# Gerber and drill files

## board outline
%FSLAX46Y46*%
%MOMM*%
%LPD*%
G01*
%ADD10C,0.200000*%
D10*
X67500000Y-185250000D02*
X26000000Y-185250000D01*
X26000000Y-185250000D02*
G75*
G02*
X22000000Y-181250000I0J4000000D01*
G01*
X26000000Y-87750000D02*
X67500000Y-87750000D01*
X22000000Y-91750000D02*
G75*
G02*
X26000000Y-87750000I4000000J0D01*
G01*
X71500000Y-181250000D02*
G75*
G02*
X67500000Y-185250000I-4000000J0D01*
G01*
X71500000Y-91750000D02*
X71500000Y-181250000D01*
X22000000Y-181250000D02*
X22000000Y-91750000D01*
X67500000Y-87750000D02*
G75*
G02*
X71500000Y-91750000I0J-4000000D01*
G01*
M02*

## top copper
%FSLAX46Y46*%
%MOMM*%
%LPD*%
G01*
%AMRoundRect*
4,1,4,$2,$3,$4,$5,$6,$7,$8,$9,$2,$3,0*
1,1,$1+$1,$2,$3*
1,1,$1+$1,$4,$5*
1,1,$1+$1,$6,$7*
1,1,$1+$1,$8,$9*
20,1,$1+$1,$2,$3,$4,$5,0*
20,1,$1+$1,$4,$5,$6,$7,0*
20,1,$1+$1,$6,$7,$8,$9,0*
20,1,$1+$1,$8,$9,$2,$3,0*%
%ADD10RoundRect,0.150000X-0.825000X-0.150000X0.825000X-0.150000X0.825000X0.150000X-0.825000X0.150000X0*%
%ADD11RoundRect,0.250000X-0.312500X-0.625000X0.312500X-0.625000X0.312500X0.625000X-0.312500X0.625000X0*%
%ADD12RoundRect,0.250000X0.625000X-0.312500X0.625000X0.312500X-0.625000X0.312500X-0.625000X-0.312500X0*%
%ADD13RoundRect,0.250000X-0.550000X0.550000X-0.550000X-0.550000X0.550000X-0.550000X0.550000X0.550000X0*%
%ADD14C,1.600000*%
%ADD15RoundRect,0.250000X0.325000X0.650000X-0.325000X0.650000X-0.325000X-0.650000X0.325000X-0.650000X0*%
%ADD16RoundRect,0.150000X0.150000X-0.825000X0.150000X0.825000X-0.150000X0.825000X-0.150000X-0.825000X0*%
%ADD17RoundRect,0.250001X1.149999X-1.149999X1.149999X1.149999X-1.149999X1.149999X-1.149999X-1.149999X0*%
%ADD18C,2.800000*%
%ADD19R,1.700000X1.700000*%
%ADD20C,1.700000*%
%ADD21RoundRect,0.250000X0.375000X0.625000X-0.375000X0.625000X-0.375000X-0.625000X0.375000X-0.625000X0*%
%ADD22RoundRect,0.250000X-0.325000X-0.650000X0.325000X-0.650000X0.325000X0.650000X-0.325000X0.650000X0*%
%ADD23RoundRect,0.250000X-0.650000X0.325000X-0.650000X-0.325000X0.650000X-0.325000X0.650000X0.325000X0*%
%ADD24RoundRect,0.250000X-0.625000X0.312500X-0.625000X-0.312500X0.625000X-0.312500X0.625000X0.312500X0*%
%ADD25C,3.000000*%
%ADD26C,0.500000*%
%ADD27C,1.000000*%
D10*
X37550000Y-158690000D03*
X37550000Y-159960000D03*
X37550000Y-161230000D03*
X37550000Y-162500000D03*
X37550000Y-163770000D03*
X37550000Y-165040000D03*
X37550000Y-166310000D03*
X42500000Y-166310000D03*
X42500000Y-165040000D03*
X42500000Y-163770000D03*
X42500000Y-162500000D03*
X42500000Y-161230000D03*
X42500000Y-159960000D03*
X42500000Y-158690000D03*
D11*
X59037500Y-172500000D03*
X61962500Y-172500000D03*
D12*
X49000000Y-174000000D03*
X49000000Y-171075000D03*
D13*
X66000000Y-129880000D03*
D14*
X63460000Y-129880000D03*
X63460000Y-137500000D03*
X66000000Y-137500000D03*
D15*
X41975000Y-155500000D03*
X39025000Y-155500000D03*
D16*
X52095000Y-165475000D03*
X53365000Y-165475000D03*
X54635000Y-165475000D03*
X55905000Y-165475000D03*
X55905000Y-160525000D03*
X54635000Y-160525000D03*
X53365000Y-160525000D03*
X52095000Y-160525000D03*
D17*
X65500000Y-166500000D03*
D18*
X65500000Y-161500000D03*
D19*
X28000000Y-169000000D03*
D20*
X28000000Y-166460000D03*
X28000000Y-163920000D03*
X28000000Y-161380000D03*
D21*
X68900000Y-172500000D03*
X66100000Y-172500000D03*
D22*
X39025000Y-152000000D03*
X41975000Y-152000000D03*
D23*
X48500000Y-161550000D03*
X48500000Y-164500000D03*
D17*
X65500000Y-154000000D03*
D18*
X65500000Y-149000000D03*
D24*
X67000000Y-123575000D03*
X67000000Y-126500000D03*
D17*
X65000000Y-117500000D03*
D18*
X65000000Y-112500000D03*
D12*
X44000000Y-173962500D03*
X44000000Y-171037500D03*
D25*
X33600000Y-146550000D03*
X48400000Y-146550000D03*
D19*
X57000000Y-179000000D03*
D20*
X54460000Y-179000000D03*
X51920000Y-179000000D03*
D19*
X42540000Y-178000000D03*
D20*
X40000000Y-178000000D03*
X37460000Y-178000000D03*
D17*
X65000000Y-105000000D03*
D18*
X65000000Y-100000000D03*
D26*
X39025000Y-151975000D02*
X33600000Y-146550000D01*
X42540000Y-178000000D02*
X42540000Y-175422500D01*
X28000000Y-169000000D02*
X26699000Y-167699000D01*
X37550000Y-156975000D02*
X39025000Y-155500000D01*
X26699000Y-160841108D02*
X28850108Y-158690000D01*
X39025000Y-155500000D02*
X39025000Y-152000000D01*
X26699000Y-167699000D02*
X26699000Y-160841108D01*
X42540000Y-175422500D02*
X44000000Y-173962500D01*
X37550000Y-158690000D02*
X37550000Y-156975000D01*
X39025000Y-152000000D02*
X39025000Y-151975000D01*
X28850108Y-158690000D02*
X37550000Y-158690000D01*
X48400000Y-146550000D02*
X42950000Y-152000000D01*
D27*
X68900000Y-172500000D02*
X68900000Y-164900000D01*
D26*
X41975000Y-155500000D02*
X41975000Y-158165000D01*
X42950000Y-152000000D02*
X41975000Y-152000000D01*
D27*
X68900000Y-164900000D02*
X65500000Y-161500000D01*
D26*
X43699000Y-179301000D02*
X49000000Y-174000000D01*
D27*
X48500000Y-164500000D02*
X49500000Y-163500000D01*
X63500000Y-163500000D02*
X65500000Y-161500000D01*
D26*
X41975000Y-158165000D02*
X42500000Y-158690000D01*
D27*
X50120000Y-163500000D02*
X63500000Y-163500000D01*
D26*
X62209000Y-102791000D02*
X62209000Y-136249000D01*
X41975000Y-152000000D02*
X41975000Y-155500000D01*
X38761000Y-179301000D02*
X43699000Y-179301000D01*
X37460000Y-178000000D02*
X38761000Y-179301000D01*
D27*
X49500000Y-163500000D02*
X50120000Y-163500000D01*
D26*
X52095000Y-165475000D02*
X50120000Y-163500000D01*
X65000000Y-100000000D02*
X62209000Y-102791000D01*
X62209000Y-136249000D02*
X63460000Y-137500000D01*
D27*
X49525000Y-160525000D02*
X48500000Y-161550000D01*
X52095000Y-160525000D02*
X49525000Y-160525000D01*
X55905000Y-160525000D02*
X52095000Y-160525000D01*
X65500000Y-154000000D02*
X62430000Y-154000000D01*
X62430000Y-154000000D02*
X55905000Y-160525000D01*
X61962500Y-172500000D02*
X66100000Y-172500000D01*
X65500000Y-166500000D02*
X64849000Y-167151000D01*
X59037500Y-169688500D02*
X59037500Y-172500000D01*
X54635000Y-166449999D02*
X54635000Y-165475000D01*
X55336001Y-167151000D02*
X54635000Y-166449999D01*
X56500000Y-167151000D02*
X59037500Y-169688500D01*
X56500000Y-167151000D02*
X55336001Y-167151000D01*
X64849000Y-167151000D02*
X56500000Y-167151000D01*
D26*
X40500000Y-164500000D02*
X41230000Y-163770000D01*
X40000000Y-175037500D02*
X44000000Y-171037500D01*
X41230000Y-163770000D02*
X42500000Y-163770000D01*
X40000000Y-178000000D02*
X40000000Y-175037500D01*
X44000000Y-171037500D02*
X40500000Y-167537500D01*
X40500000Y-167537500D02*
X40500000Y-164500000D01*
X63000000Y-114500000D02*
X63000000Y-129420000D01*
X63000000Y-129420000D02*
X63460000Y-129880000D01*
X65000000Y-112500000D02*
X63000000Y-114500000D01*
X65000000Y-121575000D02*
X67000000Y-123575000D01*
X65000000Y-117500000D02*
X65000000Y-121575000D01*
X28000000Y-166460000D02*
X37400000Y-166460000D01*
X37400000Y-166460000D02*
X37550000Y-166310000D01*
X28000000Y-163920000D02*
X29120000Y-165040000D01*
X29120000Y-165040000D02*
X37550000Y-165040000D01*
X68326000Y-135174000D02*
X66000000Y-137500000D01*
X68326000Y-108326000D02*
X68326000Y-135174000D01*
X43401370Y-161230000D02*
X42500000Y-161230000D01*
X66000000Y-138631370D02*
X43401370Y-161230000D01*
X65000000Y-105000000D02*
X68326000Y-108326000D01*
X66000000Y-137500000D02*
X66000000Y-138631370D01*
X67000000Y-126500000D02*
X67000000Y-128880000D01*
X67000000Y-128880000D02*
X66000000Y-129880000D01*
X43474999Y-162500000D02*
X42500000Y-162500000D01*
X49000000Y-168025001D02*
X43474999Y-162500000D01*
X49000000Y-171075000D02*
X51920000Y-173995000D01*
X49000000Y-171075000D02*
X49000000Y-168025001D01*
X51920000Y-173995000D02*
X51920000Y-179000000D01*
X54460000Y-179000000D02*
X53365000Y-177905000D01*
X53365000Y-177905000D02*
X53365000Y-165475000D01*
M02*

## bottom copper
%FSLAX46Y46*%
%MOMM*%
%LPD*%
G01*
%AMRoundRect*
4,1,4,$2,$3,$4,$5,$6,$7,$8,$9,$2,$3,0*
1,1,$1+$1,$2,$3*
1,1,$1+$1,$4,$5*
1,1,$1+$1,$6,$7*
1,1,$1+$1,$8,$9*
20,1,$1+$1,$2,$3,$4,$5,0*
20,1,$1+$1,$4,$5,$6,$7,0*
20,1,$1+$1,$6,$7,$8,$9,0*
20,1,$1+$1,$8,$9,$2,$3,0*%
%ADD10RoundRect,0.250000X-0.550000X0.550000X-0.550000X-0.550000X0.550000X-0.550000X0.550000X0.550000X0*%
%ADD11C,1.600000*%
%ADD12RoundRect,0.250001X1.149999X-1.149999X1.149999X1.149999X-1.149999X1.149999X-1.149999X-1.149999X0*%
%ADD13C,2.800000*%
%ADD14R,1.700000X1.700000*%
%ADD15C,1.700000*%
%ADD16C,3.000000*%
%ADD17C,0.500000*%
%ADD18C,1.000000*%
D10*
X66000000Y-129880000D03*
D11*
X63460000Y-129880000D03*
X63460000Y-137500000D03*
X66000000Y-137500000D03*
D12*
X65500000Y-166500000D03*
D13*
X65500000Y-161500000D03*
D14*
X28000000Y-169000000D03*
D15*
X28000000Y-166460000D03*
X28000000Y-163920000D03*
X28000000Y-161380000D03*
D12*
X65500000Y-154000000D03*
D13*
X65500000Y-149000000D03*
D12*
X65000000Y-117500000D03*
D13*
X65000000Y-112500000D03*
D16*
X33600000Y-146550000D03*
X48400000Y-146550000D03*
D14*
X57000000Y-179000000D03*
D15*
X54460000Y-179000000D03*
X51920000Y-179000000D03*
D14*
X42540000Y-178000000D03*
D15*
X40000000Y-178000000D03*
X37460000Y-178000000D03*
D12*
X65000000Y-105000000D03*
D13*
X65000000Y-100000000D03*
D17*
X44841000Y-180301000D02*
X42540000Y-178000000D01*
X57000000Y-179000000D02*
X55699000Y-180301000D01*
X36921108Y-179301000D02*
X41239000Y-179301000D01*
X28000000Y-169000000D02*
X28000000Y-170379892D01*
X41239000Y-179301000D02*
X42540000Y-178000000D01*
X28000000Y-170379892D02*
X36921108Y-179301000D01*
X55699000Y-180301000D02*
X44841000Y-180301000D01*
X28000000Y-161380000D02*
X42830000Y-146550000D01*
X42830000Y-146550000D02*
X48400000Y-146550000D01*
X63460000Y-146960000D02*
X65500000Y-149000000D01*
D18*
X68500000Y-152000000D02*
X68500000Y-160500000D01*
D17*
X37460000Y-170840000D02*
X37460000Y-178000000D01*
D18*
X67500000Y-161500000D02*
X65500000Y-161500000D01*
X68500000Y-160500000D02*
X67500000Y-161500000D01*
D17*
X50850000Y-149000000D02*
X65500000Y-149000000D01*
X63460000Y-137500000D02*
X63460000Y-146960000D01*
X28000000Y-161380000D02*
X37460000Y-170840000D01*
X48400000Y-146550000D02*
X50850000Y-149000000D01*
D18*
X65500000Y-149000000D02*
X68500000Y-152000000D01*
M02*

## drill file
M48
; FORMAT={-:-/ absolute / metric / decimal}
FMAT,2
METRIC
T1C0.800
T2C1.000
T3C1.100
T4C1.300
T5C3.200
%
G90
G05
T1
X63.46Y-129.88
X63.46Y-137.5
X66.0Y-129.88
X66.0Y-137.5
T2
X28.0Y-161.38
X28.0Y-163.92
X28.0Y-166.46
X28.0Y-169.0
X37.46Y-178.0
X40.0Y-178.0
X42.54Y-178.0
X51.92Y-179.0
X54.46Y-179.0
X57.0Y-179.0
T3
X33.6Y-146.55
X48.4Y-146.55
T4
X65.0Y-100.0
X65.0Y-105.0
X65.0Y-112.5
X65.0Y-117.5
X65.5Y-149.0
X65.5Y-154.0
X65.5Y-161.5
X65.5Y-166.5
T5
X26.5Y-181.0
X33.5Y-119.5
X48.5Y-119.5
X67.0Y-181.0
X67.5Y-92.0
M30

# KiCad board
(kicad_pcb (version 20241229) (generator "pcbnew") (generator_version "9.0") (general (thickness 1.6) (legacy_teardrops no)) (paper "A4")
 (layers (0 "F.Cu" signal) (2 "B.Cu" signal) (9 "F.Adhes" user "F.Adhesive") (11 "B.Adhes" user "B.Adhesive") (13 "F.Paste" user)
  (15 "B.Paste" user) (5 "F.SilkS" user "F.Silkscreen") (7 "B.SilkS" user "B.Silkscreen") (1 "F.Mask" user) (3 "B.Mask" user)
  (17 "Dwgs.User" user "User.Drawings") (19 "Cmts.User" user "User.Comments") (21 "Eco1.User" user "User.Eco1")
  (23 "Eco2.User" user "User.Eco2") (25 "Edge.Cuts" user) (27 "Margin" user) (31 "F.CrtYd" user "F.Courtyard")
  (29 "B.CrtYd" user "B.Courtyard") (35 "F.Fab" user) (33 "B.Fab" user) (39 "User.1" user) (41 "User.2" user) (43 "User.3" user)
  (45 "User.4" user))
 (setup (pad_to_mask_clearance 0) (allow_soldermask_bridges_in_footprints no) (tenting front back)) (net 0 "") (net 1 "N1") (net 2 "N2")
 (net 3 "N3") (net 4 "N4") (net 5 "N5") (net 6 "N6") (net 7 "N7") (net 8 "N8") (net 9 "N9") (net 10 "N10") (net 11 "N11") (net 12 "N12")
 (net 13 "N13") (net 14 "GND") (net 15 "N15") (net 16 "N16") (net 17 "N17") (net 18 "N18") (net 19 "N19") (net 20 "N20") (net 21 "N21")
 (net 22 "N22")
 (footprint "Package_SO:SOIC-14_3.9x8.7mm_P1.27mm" (layer "F.Cu") (at 40.025 162.5)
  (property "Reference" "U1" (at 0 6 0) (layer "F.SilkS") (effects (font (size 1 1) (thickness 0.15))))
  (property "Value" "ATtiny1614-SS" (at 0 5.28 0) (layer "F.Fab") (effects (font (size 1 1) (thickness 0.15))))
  (pad "1" smd roundrect (at -2.475 -3.81) (size 1.95 0.6) (layers "F.Cu" "F.Mask" "F.Paste") (roundrect_rratio 0.25) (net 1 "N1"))
  (pad "2" smd roundrect (at -2.475 -2.54) (size 1.95 0.6) (layers "F.Cu" "F.Mask" "F.Paste") (roundrect_rratio 0.25) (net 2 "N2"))
  (pad "3" smd roundrect (at -2.475 -1.27) (size 1.95 0.6) (layers "F.Cu" "F.Mask" "F.Paste") (roundrect_rratio 0.25) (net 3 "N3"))
  (pad "4" smd roundrect (at -2.475 0) (size 1.95 0.6) (layers "F.Cu" "F.Mask" "F.Paste") (roundrect_rratio 0.25) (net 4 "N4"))
  (pad "5" smd roundrect (at -2.475 1.27) (size 1.95 0.6) (layers "F.Cu" "F.Mask" "F.Paste") (roundrect_rratio 0.25) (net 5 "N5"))
  (pad "6" smd roundrect (at -2.475 2.54) (size 1.95 0.6) (layers "F.Cu" "F.Mask" "F.Paste") (roundrect_rratio 0.25) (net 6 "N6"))
  (pad "7" smd roundrect (at -2.475 3.81) (size 1.95 0.6) (layers "F.Cu" "F.Mask" "F.Paste") (roundrect_rratio 0.25) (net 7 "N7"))
  (pad "8" smd roundrect (at 2.475 3.81) (size 1.95 0.6) (layers "F.Cu" "F.Mask" "F.Paste") (roundrect_rratio 0.25) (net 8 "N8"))
  (pad "9" smd roundrect (at 2.475 2.54) (size 1.95 0.6) (layers "F.Cu" "F.Mask" "F.Paste") (roundrect_rratio 0.25) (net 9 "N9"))
  (pad "10" smd roundrect (at 2.475 1.27) (size 1.95 0.6) (layers "F.Cu" "F.Mask" "F.Paste") (roundrect_rratio 0.25) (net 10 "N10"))
  (pad "11" smd roundrect (at 2.475 0) (size 1.95 0.6) (layers "F.Cu" "F.Mask" "F.Paste") (roundrect_rratio 0.25) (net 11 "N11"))
  (pad "12" smd roundrect (at 2.475 -1.27) (size 1.95 0.6) (layers "F.Cu" "F.Mask" "F.Paste") (roundrect_rratio 0.25) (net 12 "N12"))
  (pad "13" smd roundrect (at 2.475 -2.54) (size 1.95 0.6) (layers "F.Cu" "F.Mask" "F.Paste") (roundrect_rratio 0.25) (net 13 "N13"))
  (pad "14" smd roundrect (at 2.475 -3.81) (size 1.95 0.6) (layers "F.Cu" "F.Mask" "F.Paste") (roundrect_rratio 0.25) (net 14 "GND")))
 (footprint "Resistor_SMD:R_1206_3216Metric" (layer "F.Cu") (at 60.5 172.5)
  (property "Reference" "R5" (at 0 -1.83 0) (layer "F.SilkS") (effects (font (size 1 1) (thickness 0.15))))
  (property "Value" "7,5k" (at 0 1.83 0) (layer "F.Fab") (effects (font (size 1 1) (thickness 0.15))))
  (pad "1" smd roundrect (at -1.4625 0) (size 1.125 1.75) (layers "F.Cu" "F.Mask" "F.Paste") (roundrect_rratio 0.222222) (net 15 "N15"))
  (pad "2" smd roundrect (at 1.4625 0) (size 1.125 1.75) (layers "F.Cu" "F.Mask" "F.Paste") (roundrect_rratio 0.222222) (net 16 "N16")))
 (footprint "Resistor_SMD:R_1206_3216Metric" (layer "F.Cu") (at 49 172.5375 90)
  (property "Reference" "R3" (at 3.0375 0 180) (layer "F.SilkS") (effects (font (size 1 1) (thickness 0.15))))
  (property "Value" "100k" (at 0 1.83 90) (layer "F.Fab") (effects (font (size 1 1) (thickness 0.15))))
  (pad "1" smd roundrect (at -1.4625 0 90) (size 1.125 1.75) (layers "F.Cu" "F.Mask" "F.Paste") (roundrect_rratio 0.222222) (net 14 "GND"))
  (pad "2" smd roundrect (at 1.4625 0 90) (size 1.125 1.75) (layers "F.Cu" "F.Mask" "F.Paste") (roundrect_rratio 0.222222) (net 11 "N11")))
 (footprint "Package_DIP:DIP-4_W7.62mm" (layer "F.Cu") (at 66 129.88 -90)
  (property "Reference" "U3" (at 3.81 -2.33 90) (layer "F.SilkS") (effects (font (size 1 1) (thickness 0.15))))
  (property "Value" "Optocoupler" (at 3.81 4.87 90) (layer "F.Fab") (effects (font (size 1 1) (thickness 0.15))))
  (pad "1" thru_hole roundrect (at 0 0 270) (size 1.6 1.6) (drill 0.8) (layers "*.Cu" "*.Mask") (remove_unused_layers no)
   (roundrect_rratio 0.15625) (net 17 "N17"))
  (pad "2" thru_hole circle (at 0 2.54 270) (size 1.6 1.6) (drill 0.8) (layers "*.Cu" "*.Mask") (remove_unused_layers no) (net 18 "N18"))
  (pad "3" thru_hole circle (at 7.62 2.54 270) (size 1.6 1.6) (drill 0.8) (layers "*.Cu" "*.Mask") (remove_unused_layers no) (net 14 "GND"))
  (pad "4" thru_hole circle (at 7.62 0 270) (size 1.6 1.6) (drill 0.8) (layers "*.Cu" "*.Mask") (remove_unused_layers no) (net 12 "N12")))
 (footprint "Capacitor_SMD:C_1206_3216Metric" (layer "F.Cu") (at 40.5 155.5 180)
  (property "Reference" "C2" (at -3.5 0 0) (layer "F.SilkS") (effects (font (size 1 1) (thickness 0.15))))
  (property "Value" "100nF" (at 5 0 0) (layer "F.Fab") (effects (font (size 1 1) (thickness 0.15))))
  (pad "1" smd roundrect (at -1.475 0 180) (size 1.15 1.8) (layers "F.Cu" "F.Mask" "F.Paste") (roundrect_rratio 0.217391) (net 14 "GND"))
  (pad "2" smd roundrect (at 1.475 0 180) (size 1.15 1.8) (layers "F.Cu" "F.Mask" "F.Paste") (roundrect_rratio 0.217391) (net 1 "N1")))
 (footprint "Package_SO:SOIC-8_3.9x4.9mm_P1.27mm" (layer "F.Cu") (at 54 163 90)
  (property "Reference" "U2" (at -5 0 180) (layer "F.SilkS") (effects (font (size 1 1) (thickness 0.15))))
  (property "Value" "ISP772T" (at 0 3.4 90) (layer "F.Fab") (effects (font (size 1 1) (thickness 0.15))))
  (pad "1" smd roundrect (at -2.475 -1.905 90) (size 1.95 0.6) (layers "F.Cu" "F.Mask" "F.Paste") (roundrect_rratio 0.25) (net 14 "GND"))
  (pad "2" smd roundrect (at -2.475 -0.635 90) (size 1.95 0.6) (layers "F.Cu" "F.Mask" "F.Paste") (roundrect_rratio 0.25) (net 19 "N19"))
  (pad "3" smd roundrect (at -2.475 0.635 90) (size 1.95 0.6) (layers "F.Cu" "F.Mask" "F.Paste") (roundrect_rratio 0.25) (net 15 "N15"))
  (pad "4" smd roundrect (at -2.475 1.905 90) (size 1.95 0.6) (layers "F.Cu" "F.Mask" "F.Paste") (roundrect_rratio 0.25) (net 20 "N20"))
  (pad "5" smd roundrect (at 2.475 1.905 90) (size 1.95 0.6) (layers "F.Cu" "F.Mask" "F.Paste") (roundrect_rratio 0.25) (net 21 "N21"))
  (pad "6" smd roundrect (at 2.475 0.635 90) (size 1.95 0.6) (layers "F.Cu" "F.Mask" "F.Paste") (roundrect_rratio 0.25) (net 21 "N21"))
  (pad "7" smd roundrect (at 2.475 -0.635 90) (size 1.95 0.6) (layers "F.Cu" "F.Mask" "F.Paste") (roundrect_rratio 0.25) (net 21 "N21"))
  (pad "8" smd roundrect (at 2.475 -1.905 90) (size 1.95 0.6) (layers "F.Cu" "F.Mask" "F.Paste") (roundrect_rratio 0.25) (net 21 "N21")))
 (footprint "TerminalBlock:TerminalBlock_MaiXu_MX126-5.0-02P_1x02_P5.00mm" (layer "F.Cu") (at 65.5 166.5 90)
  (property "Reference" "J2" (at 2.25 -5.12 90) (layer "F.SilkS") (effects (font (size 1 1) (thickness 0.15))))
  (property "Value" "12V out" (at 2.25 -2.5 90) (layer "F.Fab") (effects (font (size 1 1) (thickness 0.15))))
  (pad "1" thru_hole roundrect (at 0 0 90) (size 2.8 2.8) (drill 1.3) (layers "*.Cu" "*.Mask") (remove_unused_layers no)
   (roundrect_rratio 0.089286) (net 15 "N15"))
  (pad "2" thru_hole circle (at 5 0 90) (size 2.8 2.8) (drill 1.3) (layers "*.Cu" "*.Mask") (remove_unused_layers no) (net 14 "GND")))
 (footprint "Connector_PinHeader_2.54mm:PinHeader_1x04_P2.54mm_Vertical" (layer "F.Cu") (at 28 169 180)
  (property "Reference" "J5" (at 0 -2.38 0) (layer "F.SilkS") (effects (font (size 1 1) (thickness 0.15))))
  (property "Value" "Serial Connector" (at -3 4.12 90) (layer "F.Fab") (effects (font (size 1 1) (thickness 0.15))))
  (pad "1" thru_hole rect (at 0 0 180) (size 1.7 1.7) (drill 1) (layers "*.Cu" "*.Mask") (remove_unused_layers no) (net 1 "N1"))
  (pad "2" thru_hole circle (at 0 2.54 180) (size 1.7 1.7) (drill 1) (layers "*.Cu" "*.Mask") (remove_unused_layers no) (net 7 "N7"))
  (pad "3" thru_hole circle (at 0 5.08 180) (size 1.7 1.7) (drill 1) (layers "*.Cu" "*.Mask") (remove_unused_layers no) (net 6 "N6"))
  (pad "4" thru_hole circle (at 0 7.62 180) (size 1.7 1.7) (drill 1) (layers "*.Cu" "*.Mask") (remove_unused_layers no) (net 14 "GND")))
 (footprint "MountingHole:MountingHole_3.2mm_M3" (layer "F.Cu") (at 67.5 92)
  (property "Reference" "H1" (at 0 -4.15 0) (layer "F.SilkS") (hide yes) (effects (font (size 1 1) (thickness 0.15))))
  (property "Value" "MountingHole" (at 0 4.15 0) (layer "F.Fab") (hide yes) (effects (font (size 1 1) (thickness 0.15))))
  (pad "" np_thru_hole circle (at 0 0) (size 3.2 3.2) (drill 3.2) (layers "*.Cu" "*.Mask")))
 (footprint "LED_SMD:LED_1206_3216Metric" (layer "F.Cu") (at 67.5 172.5 180)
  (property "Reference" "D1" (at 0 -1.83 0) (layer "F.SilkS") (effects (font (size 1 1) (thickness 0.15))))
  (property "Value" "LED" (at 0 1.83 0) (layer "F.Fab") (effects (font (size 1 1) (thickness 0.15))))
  (pad "1" smd roundrect (at -1.4 0 180) (size 1.25 1.75) (layers "F.Cu" "F.Mask" "F.Paste") (roundrect_rratio 0.2) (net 14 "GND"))
  (pad "2" smd roundrect (at 1.4 0 180) (size 1.25 1.75) (layers "F.Cu" "F.Mask" "F.Paste") (roundrect_rratio 0.2) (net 16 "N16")))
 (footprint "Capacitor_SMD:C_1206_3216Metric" (layer "F.Cu") (at 40.5 152)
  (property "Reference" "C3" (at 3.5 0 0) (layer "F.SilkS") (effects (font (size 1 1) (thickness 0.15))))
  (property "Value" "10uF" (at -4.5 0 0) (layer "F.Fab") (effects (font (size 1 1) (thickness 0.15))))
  (pad "1" smd roundrect (at -1.475 0) (size 1.15 1.8) (layers "F.Cu" "F.Mask" "F.Paste") (roundrect_rratio 0.217391) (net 1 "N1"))
  (pad "2" smd roundrect (at 1.475 0) (size 1.15 1.8) (layers "F.Cu" "F.Mask" "F.Paste") (roundrect_rratio 0.217391) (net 14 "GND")))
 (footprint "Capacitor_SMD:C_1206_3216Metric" (layer "F.Cu") (at 48.5 163.025 -90)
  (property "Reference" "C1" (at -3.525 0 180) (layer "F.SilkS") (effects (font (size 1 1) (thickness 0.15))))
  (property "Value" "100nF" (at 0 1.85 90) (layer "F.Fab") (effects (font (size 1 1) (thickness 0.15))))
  (pad "1" smd roundrect (at -1.475 0 270) (size 1.15 1.8) (layers "F.Cu" "F.Mask" "F.Paste") (roundrect_rratio 0.217391) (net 21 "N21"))
  (pad "2" smd roundrect (at 1.475 0 270) (size 1.15 1.8) (layers "F.Cu" "F.Mask" "F.Paste") (roundrect_rratio 0.217391) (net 14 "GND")))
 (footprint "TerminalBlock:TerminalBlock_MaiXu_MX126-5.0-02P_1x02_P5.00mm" (layer "F.Cu") (at 65.5 154 90)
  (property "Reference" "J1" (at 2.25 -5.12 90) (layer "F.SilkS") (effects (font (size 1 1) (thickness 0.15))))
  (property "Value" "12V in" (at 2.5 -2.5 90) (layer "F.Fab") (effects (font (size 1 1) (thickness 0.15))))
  (pad "1" thru_hole roundrect (at 0 0 90) (size 2.8 2.8) (drill 1.3) (layers "*.Cu" "*.Mask") (remove_unused_layers no)
   (roundrect_rratio 0.089286) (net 21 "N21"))
  (pad "2" thru_hole circle (at 5 0 90) (size 2.8 2.8) (drill 1.3) (layers "*.Cu" "*.Mask") (remove_unused_layers no) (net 14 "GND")))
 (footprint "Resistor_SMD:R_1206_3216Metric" (layer "F.Cu") (at 67 125.0375 -90)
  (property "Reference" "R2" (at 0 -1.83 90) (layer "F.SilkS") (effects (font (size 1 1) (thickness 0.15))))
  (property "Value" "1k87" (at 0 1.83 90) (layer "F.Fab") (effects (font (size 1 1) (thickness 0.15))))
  (pad "1" smd roundrect (at -1.4625 0 270) (size 1.125 1.75) (layers "F.Cu" "F.Mask" "F.Paste") (roundrect_rratio 0.222222) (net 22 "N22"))
  (pad "2" smd roundrect (at 1.4625 0 270) (size 1.125 1.75) (layers "F.Cu" "F.Mask" "F.Paste") (roundrect_rratio 0.222222) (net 17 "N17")))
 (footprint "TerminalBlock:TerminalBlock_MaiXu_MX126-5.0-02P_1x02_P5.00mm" (layer "F.Cu") (at 65 117.5 90)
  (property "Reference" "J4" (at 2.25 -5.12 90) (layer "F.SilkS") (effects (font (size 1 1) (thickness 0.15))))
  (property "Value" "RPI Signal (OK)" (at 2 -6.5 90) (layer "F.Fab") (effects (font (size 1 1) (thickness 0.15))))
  (pad "1" thru_hole roundrect (at 0 0 90) (size 2.8 2.8) (drill 1.3) (layers "*.Cu" "*.Mask") (remove_unused_layers no)
   (roundrect_rratio 0.089286) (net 22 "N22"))
  (pad "2" thru_hole circle (at 5 0 90) (size 2.8 2.8) (drill 1.3) (layers "*.Cu" "*.Mask") (remove_unused_layers no) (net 18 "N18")))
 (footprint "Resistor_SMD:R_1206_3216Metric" (layer "F.Cu") (at 44 172.5 90)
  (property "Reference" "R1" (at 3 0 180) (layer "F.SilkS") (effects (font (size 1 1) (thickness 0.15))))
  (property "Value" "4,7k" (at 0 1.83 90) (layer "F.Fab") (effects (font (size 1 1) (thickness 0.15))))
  (pad "1" smd roundrect (at -1.4625 0 90) (size 1.125 1.75) (layers "F.Cu" "F.Mask" "F.Paste") (roundrect_rratio 0.222222) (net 1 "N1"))
  (pad "2" smd roundrect (at 1.4625 0 90) (size 1.125 1.75) (layers "F.Cu" "F.Mask" "F.Paste") (roundrect_rratio 0.222222) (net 10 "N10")))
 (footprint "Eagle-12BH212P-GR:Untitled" (layer "F.Cu") (at 41 153.55)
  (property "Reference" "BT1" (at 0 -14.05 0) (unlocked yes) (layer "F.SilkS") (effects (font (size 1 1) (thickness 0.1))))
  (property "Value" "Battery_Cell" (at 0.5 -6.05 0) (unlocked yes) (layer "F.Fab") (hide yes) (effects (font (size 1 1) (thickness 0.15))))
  (pad "" np_thru_hole circle (at -7.5 -34.05) (size 1 1) (drill 3.2) (layers "*.Cu" "*.Mask"))
  (pad "" np_thru_hole circle (at 7.5 -34.05) (size 1 1) (drill 3.2) (layers "*.Cu" "*.Mask"))
  (pad "1" thru_hole circle (at -7.4 -7) (size 3 3) (drill 1.1) (layers "*.Cu" "*.Mask") (remove_unused_layers no) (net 1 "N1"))
  (pad "2" thru_hole circle (at 7.4 -7) (size 3 3) (drill 1.1) (layers "*.Cu" "*.Mask") (remove_unused_layers no) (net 14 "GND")))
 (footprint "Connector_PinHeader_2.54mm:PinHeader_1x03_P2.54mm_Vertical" (layer "F.Cu") (at 57 179 -90)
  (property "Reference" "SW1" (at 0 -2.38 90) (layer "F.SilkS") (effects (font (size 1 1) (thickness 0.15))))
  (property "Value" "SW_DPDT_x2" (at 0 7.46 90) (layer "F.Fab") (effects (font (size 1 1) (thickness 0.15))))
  (pad "1" thru_hole rect (at 0 0 270) (size 1.7 1.7) (drill 1) (layers "*.Cu" "*.Mask") (remove_unused_layers no) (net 1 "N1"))
  (pad "2" thru_hole circle (at 0 2.54 270) (size 1.7 1.7) (drill 1) (layers "*.Cu" "*.Mask") (remove_unused_layers no) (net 19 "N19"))
  (pad "3" thru_hole circle (at 0 5.08 270) (size 1.7 1.7) (drill 1) (layers "*.Cu" "*.Mask") (remove_unused_layers no) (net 11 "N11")))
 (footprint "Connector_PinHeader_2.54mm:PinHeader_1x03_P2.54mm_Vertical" (layer "F.Cu") (at 42.54 178 -90)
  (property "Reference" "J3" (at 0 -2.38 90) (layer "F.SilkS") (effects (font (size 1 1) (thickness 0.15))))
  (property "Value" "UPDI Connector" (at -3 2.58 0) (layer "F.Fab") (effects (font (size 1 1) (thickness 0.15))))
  (pad "1" thru_hole rect (at 0 0 270) (size 1.7 1.7) (drill 1) (layers "*.Cu" "*.Mask") (remove_unused_layers no) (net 1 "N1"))
  (pad "2" thru_hole circle (at 0 2.54 270) (size 1.7 1.7) (drill 1) (layers "*.Cu" "*.Mask") (remove_unused_layers no) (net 10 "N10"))
  (pad "3" thru_hole circle (at 0 5.08 270) (size 1.7 1.7) (drill 1) (layers "*.Cu" "*.Mask") (remove_unused_layers no) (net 14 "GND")))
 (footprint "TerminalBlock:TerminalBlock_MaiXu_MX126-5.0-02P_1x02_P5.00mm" (layer "F.Cu") (at 65 105 90)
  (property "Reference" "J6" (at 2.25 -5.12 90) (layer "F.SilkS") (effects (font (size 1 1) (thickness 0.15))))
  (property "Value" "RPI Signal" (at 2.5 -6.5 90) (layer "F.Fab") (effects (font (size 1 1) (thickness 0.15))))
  (pad "1" thru_hole roundrect (at 0 0 90) (size 2.8 2.8) (drill 1.3) (layers "*.Cu" "*.Mask") (remove_unused_layers no)
   (roundrect_rratio 0.089286) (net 12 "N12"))
  (pad "2" thru_hole circle (at 5 0 90) (size 2.8 2.8) (drill 1.3) (layers "*.Cu" "*.Mask") (remove_unused_layers no) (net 14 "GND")))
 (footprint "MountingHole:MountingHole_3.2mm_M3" (layer "F.Cu") (at 26.5 181)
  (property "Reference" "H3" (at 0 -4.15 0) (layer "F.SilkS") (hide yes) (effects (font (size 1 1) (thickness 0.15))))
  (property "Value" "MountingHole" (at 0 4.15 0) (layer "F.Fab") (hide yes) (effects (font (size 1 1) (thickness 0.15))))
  (pad "" np_thru_hole circle (at 0 0) (size 3.2 3.2) (drill 3.2) (layers "*.Cu" "*.Mask")))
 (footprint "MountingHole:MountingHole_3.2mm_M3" (layer "F.Cu") (at 67 181)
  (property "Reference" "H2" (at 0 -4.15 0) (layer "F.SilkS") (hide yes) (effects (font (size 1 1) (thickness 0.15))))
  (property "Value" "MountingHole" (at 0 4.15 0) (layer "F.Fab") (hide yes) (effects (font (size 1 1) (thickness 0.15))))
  (pad "" np_thru_hole circle (at 0 0) (size 3.2 3.2) (drill 3.2) (layers "*.Cu" "*.Mask")))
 (gr_line (start 67.5 185.25) (end 26 185.25) (stroke (width 0.2) (type default)) (layer "Edge.Cuts"))
 (gr_arc (start 26 185.25) (mid 23.171573 184.078427) (end 22 181.25) (stroke (width 0.2) (type default)) (layer "Edge.Cuts"))
 (gr_line (start 26 87.75) (end 67.5 87.75) (stroke (width 0.2) (type default)) (layer "Edge.Cuts"))
 (gr_arc (start 22 91.75) (mid 23.171573 88.921573) (end 26 87.75) (stroke (width 0.2) (type default)) (layer "Edge.Cuts"))
 (gr_arc (start 71.5 181.25) (mid 70.328427 184.078427) (end 67.5 185.25) (stroke (width 0.2) (type default)) (layer "Edge.Cuts"))
 (gr_line (start 71.5 91.75) (end 71.5 181.25) (stroke (width 0.2) (type default)) (layer "Edge.Cuts"))
 (gr_line (start 22 181.25) (end 22 91.75) (stroke (width 0.2) (type default)) (layer "Edge.Cuts"))
 (gr_arc (start 67.5 87.75) (mid 70.328427 88.921573) (end 71.5 91.75) (stroke (width 0.2) (type default)) (layer "Edge.Cuts"))
 (segment (start 39.025 151.975) (end 33.6 146.55) (width 0.5) (layer "F.Cu") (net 1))
 (segment (start 42.54 178) (end 42.54 175.4225) (width 0.5) (layer "F.Cu") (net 1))
 (segment (start 28 169) (end 26.699 167.699) (width 0.5) (layer "F.Cu") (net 1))
 (segment (start 37.55 156.975) (end 39.025 155.5) (width 0.5) (layer "F.Cu") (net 1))
 (segment (start 26.699 160.841108) (end 28.850108 158.69) (width 0.5) (layer "F.Cu") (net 1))
 (segment (start 39.025 155.5) (end 39.025 152) (width 0.5) (layer "F.Cu") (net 1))
 (segment (start 26.699 167.699) (end 26.699 160.841108) (width 0.5) (layer "F.Cu") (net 1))
 (segment (start 42.54 175.4225) (end 44 173.9625) (width 0.5) (layer "F.Cu") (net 1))
 (segment (start 37.55 158.69) (end 37.55 156.975) (width 0.5) (layer "F.Cu") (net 1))
 (segment (start 39.025 152) (end 39.025 151.975) (width 0.5) (layer "F.Cu") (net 1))
 (segment (start 28.850108 158.69) (end 37.55 158.69) (width 0.5) (layer "F.Cu") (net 1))
 (segment (start 44.841 180.301) (end 42.54 178) (width 0.5) (layer "B.Cu") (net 1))
 (segment (start 57 179) (end 55.699 180.301) (width 0.5) (layer "B.Cu") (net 1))
 (segment (start 36.921108 179.301) (end 41.239 179.301) (width 0.5) (layer "B.Cu") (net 1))
 (segment (start 28 169) (end 28 170.379892) (width 0.5) (layer "B.Cu") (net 1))
 (segment (start 41.239 179.301) (end 42.54 178) (width 0.5) (layer "B.Cu") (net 1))
 (segment (start 28 170.379892) (end 36.921108 179.301) (width 0.5) (layer "B.Cu") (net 1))
 (segment (start 55.699 180.301) (end 44.841 180.301) (width 0.5) (layer "B.Cu") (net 1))
 (segment (start 48.4 146.55) (end 42.95 152) (width 0.5) (layer "F.Cu") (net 14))
 (segment (start 68.9 172.5) (end 68.9 164.9) (width 1) (layer "F.Cu") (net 14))
 (segment (start 41.975 155.5) (end 41.975 158.165) (width 0.5) (layer "F.Cu") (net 14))
 (segment (start 42.95 152) (end 41.975 152) (width 0.5) (layer "F.Cu") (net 14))
 (segment (start 68.9 164.9) (end 65.5 161.5) (width 1) (layer "F.Cu") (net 14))
 (segment (start 43.699 179.301) (end 49 174) (width 0.5) (layer "F.Cu") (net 14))
 (segment (start 48.5 164.5) (end 49.5 163.5) (width 1) (layer "F.Cu") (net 14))
 (segment (start 63.5 163.5) (end 65.5 161.5) (width 1) (layer "F.Cu") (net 14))
 (segment (start 41.975 158.165) (end 42.5 158.69) (width 0.5) (layer "F.Cu") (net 14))
 (segment (start 50.12 163.5) (end 63.5 163.5) (width 1) (layer "F.Cu") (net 14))
 (segment (start 62.209 102.791) (end 62.209 136.249) (width 0.5) (layer "F.Cu") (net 14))
 (segment (start 41.975 152) (end 41.975 155.5) (width 0.5) (layer "F.Cu") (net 14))
 (segment (start 38.761 179.301) (end 43.699 179.301) (width 0.5) (layer "F.Cu") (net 14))
 (segment (start 37.46 178) (end 38.761 179.301) (width 0.5) (layer "F.Cu") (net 14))
 (segment (start 49.5 163.5) (end 50.12 163.5) (width 1) (layer "F.Cu") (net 14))
 (segment (start 52.095 165.475) (end 50.12 163.5) (width 0.5) (layer "F.Cu") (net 14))
 (segment (start 65 100) (end 62.209 102.791) (width 0.5) (layer "F.Cu") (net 14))
 (segment (start 62.209 136.249) (end 63.46 137.5) (width 0.5) (layer "F.Cu") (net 14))
 (segment (start 28 161.38) (end 42.83 146.55) (width 0.5) (layer "B.Cu") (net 14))
 (segment (start 42.83 146.55) (end 48.4 146.55) (width 0.5) (layer "B.Cu") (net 14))
 (segment (start 63.46 146.96) (end 65.5 149) (width 0.5) (layer "B.Cu") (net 14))
 (segment (start 68.5 152) (end 68.5 160.5) (width 1) (layer "B.Cu") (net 14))
 (segment (start 37.46 170.84) (end 37.46 178) (width 0.5) (layer "B.Cu") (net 14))
 (segment (start 67.5 161.5) (end 65.5 161.5) (width 1) (layer "B.Cu") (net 14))
 (segment (start 68.5 160.5) (end 67.5 161.5) (width 1) (layer "B.Cu") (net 14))
 (segment (start 50.85 149) (end 65.5 149) (width 0.5) (layer "B.Cu") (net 14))
 (segment (start 63.46 137.5) (end 63.46 146.96) (width 0.5) (layer "B.Cu") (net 14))
 (segment (start 28 161.38) (end 37.46 170.84) (width 0.5) (layer "B.Cu") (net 14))
 (segment (start 48.4 146.55) (end 50.85 149) (width 0.5) (layer "B.Cu") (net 14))
 (segment (start 65.5 149) (end 68.5 152) (width 1) (layer "B.Cu") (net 14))
 (segment (start 49.525 160.525) (end 48.5 161.55) (width 1) (layer "F.Cu") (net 21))
 (segment (start 52.095 160.525) (end 49.525 160.525) (width 1) (layer "F.Cu") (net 21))
 (segment (start 55.905 160.525) (end 52.095 160.525) (width 1) (layer "F.Cu") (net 21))
 (segment (start 65.5 154) (end 62.43 154) (width 1) (layer "F.Cu") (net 21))
 (segment (start 62.43 154) (end 55.905 160.525) (width 1) (layer "F.Cu") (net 21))
 (segment (start 61.9625 172.5) (end 66.1 172.5) (width 1) (layer "F.Cu") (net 16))
 (segment (start 65.5 166.5) (end 64.849 167.151) (width 1) (layer "F.Cu") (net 15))
 (segment (start 59.0375 169.6885) (end 59.0375 172.5) (width 1) (layer "F.Cu") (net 15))
 (segment (start 54.635 166.449999) (end 54.635 165.475) (width 1) (layer "F.Cu") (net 15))
 (segment (start 55.336001 167.151) (end 54.635 166.449999) (width 1) (layer "F.Cu") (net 15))
 (segment (start 56.5 167.151) (end 59.0375 169.6885) (width 1) (layer "F.Cu") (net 15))
 (segment (start 56.5 167.151) (end 55.336001 167.151) (width 1) (layer "F.Cu") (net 15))
 (segment (start 64.849 167.151) (end 56.5 167.151) (width 1) (layer "F.Cu") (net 15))
 (segment (start 40.5 164.5) (end 41.23 163.77) (width 0.5) (layer "F.Cu") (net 10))
 (segment (start 40 175.0375) (end 44 171.0375) (width 0.5) (layer "F.Cu") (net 10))
 (segment (start 41.23 163.77) (end 42.5 163.77) (width 0.5) (layer "F.Cu") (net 10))
 (segment (start 40 178) (end 40 175.0375) (width 0.5) (layer "F.Cu") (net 10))
 (segment (start 44 171.0375) (end 40.5 167.5375) (width 0.5) (layer "F.Cu") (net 10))
 (segment (start 40.5 167.5375) (end 40.5 164.5) (width 0.5) (layer "F.Cu") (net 10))
 (segment (start 63 114.5) (end 63 129.42) (width 0.5) (layer "F.Cu") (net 18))
 (segment (start 63 129.42) (end 63.46 129.88) (width 0.5) (layer "F.Cu") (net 18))
 (segment (start 65 112.5) (end 63 114.5) (width 0.5) (layer "F.Cu") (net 18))
 (segment (start 65 121.575) (end 67 123.575) (width 0.5) (layer "F.Cu") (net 22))
 (segment (start 65 117.5) (end 65 121.575) (width 0.5) (layer "F.Cu") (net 22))
 (segment (start 28 166.46) (end 37.4 166.46) (width 0.5) (layer "F.Cu") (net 7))
 (segment (start 37.4 166.46) (end 37.55 166.31) (width 0.5) (layer "F.Cu") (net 7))
 (segment (start 28 163.92) (end 29.12 165.04) (width 0.5) (layer "F.Cu") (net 6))
 (segment (start 29.12 165.04) (end 37.55 165.04) (width 0.5) (layer "F.Cu") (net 6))
 (segment (start 68.326 135.174) (end 66 137.5) (width 0.5) (layer "F.Cu") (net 12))
 (segment (start 68.326 108.326) (end 68.326 135.174) (width 0.5) (layer "F.Cu") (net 12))
 (segment (start 43.40137 161.23) (end 42.5 161.23) (width 0.5) (layer "F.Cu") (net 12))
 (segment (start 66 138.63137) (end 43.40137 161.23) (width 0.5) (layer "F.Cu") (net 12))
 (segment (start 65 105) (end 68.326 108.326) (width 0.5) (layer "F.Cu") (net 12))
 (segment (start 66 137.5) (end 66 138.63137) (width 0.5) (layer "F.Cu") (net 12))
 (segment (start 67 126.5) (end 67 128.88) (width 0.5) (layer "F.Cu") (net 17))
 (segment (start 67 128.88) (end 66 129.88) (width 0.5) (layer "F.Cu") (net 17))
 (segment (start 43.474999 162.5) (end 42.5 162.5) (width 0.5) (layer "F.Cu") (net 11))
 (segment (start 49 168.025001) (end 43.474999 162.5) (width 0.5) (layer "F.Cu") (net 11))
 (segment (start 49 171.075) (end 51.92 173.995) (width 0.5) (layer "F.Cu") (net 11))
 (segment (start 49 171.075) (end 49 168.025001) (width 0.5) (layer "F.Cu") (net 11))
 (segment (start 51.92 173.995) (end 51.92 179) (width 0.5) (layer "F.Cu") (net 11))
 (segment (start 54.46 179) (end 53.365 177.905) (width 0.5) (layer "F.Cu") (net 19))
 (segment (start 53.365 177.905) (end 53.365 165.475) (width 0.5) (layer "F.Cu") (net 19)))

